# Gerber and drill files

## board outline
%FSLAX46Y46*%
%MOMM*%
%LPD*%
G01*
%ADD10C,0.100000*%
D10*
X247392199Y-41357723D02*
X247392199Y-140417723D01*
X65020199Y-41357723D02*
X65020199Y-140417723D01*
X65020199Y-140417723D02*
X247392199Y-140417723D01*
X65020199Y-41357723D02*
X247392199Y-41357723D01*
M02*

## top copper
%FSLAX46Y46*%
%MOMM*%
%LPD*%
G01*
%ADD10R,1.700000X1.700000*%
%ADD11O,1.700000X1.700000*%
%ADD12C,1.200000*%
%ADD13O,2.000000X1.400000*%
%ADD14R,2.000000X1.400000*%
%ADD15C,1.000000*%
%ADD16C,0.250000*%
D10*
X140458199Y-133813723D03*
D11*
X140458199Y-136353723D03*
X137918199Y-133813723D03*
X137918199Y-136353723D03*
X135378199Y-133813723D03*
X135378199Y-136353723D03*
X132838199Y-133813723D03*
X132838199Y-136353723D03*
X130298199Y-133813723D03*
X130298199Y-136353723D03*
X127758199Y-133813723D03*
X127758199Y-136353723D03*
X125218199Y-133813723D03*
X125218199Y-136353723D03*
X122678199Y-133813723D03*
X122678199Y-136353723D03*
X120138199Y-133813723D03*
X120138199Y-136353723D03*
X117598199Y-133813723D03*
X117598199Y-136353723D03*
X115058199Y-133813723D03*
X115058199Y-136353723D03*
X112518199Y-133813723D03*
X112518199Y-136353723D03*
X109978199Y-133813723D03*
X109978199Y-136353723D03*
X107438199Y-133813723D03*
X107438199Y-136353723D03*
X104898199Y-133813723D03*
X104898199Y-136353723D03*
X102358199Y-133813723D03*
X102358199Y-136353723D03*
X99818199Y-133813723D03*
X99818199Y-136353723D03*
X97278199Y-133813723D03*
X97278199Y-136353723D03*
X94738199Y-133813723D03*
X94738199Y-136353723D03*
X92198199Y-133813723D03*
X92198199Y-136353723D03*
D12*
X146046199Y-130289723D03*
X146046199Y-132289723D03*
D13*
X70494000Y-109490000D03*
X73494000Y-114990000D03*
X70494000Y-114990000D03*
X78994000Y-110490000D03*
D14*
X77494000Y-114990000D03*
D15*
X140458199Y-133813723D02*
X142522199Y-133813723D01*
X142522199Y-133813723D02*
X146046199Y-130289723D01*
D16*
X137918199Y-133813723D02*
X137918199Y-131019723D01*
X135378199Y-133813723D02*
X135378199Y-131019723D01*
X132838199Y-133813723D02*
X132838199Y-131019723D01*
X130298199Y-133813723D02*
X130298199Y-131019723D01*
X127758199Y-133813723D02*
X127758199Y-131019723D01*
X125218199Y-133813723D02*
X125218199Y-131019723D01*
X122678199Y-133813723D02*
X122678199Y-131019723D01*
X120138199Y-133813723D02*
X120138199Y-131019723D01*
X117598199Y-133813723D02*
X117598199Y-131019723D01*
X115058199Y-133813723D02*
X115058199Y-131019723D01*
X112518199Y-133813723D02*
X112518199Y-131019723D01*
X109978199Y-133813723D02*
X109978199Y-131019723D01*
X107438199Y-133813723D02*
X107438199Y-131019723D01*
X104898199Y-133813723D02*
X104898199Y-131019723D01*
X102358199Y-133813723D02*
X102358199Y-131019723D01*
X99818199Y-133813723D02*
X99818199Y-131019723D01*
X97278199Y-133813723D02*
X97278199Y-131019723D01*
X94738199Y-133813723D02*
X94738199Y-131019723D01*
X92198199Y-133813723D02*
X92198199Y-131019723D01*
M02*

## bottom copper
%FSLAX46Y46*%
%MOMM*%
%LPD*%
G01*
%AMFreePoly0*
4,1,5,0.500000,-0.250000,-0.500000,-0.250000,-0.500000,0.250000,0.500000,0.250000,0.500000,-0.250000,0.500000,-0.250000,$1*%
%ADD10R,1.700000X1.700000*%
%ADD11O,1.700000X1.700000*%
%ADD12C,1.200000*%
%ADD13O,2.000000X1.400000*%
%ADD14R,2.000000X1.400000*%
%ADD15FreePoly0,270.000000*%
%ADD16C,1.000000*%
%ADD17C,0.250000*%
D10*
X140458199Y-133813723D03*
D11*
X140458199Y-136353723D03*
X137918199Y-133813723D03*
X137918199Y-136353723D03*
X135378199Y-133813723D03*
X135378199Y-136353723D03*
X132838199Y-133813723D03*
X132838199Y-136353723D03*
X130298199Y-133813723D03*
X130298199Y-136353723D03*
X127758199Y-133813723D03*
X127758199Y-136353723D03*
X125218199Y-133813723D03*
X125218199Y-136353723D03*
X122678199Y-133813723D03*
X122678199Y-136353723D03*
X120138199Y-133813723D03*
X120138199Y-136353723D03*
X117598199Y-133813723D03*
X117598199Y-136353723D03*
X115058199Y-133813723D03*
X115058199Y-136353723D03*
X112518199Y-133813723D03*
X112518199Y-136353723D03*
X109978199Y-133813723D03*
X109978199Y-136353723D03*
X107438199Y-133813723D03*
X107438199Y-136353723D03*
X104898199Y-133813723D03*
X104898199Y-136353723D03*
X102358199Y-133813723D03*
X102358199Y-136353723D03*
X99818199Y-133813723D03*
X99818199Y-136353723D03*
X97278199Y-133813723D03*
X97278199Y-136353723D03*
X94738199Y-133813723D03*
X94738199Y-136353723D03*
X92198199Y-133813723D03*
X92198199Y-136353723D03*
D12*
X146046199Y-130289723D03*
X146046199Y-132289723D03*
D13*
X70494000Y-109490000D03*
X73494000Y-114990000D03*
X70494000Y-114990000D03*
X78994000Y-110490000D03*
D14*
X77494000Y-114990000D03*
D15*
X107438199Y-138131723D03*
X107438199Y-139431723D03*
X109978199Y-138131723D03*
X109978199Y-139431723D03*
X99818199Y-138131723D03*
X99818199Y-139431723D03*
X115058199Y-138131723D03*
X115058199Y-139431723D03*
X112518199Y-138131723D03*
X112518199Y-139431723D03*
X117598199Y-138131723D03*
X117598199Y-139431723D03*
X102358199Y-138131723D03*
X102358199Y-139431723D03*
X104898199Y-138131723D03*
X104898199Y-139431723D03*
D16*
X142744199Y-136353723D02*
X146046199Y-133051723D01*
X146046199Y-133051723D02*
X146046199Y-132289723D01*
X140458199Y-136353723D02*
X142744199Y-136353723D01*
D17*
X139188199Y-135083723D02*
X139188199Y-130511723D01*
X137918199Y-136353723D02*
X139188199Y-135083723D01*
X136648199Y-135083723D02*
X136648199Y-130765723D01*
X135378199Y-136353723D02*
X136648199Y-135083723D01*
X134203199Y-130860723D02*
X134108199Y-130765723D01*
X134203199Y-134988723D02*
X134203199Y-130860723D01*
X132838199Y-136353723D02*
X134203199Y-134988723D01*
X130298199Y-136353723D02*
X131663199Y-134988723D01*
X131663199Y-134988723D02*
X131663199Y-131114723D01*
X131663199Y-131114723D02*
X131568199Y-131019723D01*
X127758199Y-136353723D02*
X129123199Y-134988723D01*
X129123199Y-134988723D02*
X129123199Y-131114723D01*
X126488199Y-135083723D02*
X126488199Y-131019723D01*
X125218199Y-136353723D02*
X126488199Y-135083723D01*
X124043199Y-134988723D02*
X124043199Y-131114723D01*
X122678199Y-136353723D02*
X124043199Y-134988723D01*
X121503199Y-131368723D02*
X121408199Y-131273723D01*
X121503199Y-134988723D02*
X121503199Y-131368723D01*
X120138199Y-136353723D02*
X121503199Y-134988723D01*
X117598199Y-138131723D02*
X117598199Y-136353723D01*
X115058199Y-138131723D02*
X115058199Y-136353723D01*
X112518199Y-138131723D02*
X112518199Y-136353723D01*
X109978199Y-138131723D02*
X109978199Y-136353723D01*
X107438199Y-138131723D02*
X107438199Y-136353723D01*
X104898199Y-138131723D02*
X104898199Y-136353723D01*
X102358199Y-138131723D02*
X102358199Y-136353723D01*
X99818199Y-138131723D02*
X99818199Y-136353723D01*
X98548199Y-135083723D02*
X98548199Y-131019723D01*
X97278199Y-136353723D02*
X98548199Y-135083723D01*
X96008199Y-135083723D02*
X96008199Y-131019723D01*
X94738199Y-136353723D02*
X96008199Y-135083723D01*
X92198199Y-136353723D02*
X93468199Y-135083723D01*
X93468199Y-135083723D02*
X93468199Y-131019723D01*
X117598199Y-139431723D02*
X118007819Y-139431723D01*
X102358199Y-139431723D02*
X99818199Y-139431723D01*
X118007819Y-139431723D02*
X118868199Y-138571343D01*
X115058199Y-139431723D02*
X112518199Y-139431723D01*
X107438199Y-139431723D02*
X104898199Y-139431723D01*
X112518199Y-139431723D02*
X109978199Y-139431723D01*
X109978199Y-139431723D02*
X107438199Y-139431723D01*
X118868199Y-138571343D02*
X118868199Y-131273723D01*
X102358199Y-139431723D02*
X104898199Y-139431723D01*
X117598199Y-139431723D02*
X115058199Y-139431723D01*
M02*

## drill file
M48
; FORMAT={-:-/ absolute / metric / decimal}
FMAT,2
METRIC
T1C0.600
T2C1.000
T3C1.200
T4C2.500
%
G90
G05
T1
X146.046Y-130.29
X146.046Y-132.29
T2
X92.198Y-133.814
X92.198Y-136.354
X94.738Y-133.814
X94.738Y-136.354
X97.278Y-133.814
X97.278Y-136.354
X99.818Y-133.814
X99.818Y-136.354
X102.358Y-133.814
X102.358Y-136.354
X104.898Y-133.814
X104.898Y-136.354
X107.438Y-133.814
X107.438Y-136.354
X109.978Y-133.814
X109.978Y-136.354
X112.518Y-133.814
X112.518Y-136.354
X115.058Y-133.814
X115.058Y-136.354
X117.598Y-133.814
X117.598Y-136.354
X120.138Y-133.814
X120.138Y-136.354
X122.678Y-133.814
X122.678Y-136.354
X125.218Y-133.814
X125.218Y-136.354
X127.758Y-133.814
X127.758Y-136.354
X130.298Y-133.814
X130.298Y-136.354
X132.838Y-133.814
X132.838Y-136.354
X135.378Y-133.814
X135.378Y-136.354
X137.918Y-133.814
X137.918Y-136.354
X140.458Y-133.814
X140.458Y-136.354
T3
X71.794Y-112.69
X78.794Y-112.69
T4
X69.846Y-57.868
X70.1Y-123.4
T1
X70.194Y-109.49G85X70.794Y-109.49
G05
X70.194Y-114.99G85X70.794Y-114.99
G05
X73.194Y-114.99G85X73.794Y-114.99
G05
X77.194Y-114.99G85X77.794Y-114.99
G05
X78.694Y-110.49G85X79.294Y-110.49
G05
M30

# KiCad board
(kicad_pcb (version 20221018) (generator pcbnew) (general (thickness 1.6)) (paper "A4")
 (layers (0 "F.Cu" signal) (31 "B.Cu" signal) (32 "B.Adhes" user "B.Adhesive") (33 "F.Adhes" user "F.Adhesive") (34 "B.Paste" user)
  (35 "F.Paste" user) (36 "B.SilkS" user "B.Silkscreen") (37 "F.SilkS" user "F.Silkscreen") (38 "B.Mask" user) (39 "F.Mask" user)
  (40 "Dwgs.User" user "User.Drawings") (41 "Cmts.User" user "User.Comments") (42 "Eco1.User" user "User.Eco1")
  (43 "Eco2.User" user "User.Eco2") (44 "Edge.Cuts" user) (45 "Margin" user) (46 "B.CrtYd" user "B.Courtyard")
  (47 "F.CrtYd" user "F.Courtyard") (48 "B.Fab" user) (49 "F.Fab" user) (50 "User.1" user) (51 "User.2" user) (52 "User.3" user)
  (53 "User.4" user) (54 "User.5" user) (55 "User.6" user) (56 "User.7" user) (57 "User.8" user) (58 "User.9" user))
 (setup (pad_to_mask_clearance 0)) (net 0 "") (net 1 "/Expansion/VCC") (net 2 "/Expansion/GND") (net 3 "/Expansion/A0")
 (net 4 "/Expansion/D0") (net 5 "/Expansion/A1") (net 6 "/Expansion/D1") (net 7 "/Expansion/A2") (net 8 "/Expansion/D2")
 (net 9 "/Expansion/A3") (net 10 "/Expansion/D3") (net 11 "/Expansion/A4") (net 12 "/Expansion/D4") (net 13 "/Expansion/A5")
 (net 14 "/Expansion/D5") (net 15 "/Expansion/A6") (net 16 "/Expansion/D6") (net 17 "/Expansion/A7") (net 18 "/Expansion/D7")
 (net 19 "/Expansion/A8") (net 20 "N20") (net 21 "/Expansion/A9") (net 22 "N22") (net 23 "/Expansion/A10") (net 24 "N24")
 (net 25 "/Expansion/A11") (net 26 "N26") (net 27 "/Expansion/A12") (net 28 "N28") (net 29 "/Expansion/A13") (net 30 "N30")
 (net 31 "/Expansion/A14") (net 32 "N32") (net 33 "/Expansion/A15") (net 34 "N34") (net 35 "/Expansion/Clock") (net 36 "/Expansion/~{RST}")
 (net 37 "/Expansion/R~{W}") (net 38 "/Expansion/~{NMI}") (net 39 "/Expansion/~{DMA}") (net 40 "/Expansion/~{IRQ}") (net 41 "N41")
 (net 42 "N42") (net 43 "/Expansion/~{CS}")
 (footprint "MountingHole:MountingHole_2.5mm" (layer "F.Cu") (at 70.100199 123.399723)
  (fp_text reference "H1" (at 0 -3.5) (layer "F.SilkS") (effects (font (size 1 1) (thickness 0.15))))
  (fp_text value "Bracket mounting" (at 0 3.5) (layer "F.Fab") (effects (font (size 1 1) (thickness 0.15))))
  (pad "" np_thru_hole circle (at 0 0) (size 2.5 2.5) (drill 2.5) (layers "*.Cu" "*.Mask")))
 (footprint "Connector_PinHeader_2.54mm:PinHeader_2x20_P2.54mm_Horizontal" (layer "F.Cu") (at 140.458199 133.813723 -90)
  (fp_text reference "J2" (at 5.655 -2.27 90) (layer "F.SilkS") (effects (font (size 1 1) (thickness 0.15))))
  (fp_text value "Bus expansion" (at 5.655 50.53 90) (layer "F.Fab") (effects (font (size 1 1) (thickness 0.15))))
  (pad "1" thru_hole rect (at 0 0 270) (size 1.7 1.7) (drill 1) (layers "*.Cu" "*.Mask") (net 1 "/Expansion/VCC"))
  (pad "2" thru_hole oval (at 2.54 0 270) (size 1.7 1.7) (drill 1) (layers "*.Cu" "*.Mask") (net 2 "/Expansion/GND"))
  (pad "3" thru_hole oval (at 0 2.54 270) (size 1.7 1.7) (drill 1) (layers "*.Cu" "*.Mask") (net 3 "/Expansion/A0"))
  (pad "4" thru_hole oval (at 2.54 2.54 270) (size 1.7 1.7) (drill 1) (layers "*.Cu" "*.Mask") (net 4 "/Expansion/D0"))
  (pad "5" thru_hole oval (at 0 5.08 270) (size 1.7 1.7) (drill 1) (layers "*.Cu" "*.Mask") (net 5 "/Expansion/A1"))
  (pad "6" thru_hole oval (at 2.54 5.08 270) (size 1.7 1.7) (drill 1) (layers "*.Cu" "*.Mask") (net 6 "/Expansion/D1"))
  (pad "7" thru_hole oval (at 0 7.62 270) (size 1.7 1.7) (drill 1) (layers "*.Cu" "*.Mask") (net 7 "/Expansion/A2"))
  (pad "8" thru_hole oval (at 2.54 7.62 270) (size 1.7 1.7) (drill 1) (layers "*.Cu" "*.Mask") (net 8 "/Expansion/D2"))
  (pad "9" thru_hole oval (at 0 10.16 270) (size 1.7 1.7) (drill 1) (layers "*.Cu" "*.Mask") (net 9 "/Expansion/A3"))
  (pad "10" thru_hole oval (at 2.54 10.16 270) (size 1.7 1.7) (drill 1) (layers "*.Cu" "*.Mask") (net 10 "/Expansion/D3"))
  (pad "11" thru_hole oval (at 0 12.7 270) (size 1.7 1.7) (drill 1) (layers "*.Cu" "*.Mask") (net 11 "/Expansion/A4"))
  (pad "12" thru_hole oval (at 2.54 12.7 270) (size 1.7 1.7) (drill 1) (layers "*.Cu" "*.Mask") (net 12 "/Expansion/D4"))
  (pad "13" thru_hole oval (at 0 15.24 270) (size 1.7 1.7) (drill 1) (layers "*.Cu" "*.Mask") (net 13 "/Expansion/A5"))
  (pad "14" thru_hole oval (at 2.54 15.24 270) (size 1.7 1.7) (drill 1) (layers "*.Cu" "*.Mask") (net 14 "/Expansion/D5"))
  (pad "15" thru_hole oval (at 0 17.78 270) (size 1.7 1.7) (drill 1) (layers "*.Cu" "*.Mask") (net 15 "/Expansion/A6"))
  (pad "16" thru_hole oval (at 2.54 17.78 270) (size 1.7 1.7) (drill 1) (layers "*.Cu" "*.Mask") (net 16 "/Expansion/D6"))
  (pad "17" thru_hole oval (at 0 20.32 270) (size 1.7 1.7) (drill 1) (layers "*.Cu" "*.Mask") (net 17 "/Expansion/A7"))
  (pad "18" thru_hole oval (at 2.54 20.32 270) (size 1.7 1.7) (drill 1) (layers "*.Cu" "*.Mask") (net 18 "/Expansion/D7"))
  (pad "19" thru_hole oval (at 0 22.86 270) (size 1.7 1.7) (drill 1) (layers "*.Cu" "*.Mask") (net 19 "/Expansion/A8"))
  (pad "20" thru_hole oval (at 2.54 22.86 270) (size 1.7 1.7) (drill 1) (layers "*.Cu" "*.Mask") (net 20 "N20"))
  (pad "21" thru_hole oval (at 0 25.4 270) (size 1.7 1.7) (drill 1) (layers "*.Cu" "*.Mask") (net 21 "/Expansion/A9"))
  (pad "22" thru_hole oval (at 2.54 25.4 270) (size 1.7 1.7) (drill 1) (layers "*.Cu" "*.Mask") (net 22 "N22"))
  (pad "23" thru_hole oval (at 0 27.94 270) (size 1.7 1.7) (drill 1) (layers "*.Cu" "*.Mask") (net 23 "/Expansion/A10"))
  (pad "24" thru_hole oval (at 2.54 27.94 270) (size 1.7 1.7) (drill 1) (layers "*.Cu" "*.Mask") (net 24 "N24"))
  (pad "25" thru_hole oval (at 0 30.48 270) (size 1.7 1.7) (drill 1) (layers "*.Cu" "*.Mask") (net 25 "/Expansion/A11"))
  (pad "26" thru_hole oval (at 2.54 30.48 270) (size 1.7 1.7) (drill 1) (layers "*.Cu" "*.Mask") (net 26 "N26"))
  (pad "27" thru_hole oval (at 0 33.02 270) (size 1.7 1.7) (drill 1) (layers "*.Cu" "*.Mask") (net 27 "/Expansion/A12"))
  (pad "28" thru_hole oval (at 2.54 33.02 270) (size 1.7 1.7) (drill 1) (layers "*.Cu" "*.Mask") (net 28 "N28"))
  (pad "29" thru_hole oval (at 0 35.56 270) (size 1.7 1.7) (drill 1) (layers "*.Cu" "*.Mask") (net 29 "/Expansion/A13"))
  (pad "30" thru_hole oval (at 2.54 35.56 270) (size 1.7 1.7) (drill 1) (layers "*.Cu" "*.Mask") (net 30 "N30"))
  (pad "31" thru_hole oval (at 0 38.1 270) (size 1.7 1.7) (drill 1) (layers "*.Cu" "*.Mask") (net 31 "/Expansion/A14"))
  (pad "32" thru_hole oval (at 2.54 38.1 270) (size 1.7 1.7) (drill 1) (layers "*.Cu" "*.Mask") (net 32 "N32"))
  (pad "33" thru_hole oval (at 0 40.64 270) (size 1.7 1.7) (drill 1) (layers "*.Cu" "*.Mask") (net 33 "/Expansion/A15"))
  (pad "34" thru_hole oval (at 2.54 40.64 270) (size 1.7 1.7) (drill 1) (layers "*.Cu" "*.Mask") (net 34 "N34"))
  (pad "35" thru_hole oval (at 0 43.18 270) (size 1.7 1.7) (drill 1) (layers "*.Cu" "*.Mask") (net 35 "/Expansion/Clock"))
  (pad "36" thru_hole oval (at 2.54 43.18 270) (size 1.7 1.7) (drill 1) (layers "*.Cu" "*.Mask") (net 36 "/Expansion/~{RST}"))
  (pad "37" thru_hole oval (at 0 45.72 270) (size 1.7 1.7) (drill 1) (layers "*.Cu" "*.Mask") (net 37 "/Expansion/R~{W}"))
  (pad "38" thru_hole oval (at 2.54 45.72 270) (size 1.7 1.7) (drill 1) (layers "*.Cu" "*.Mask") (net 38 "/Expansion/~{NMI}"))
  (pad "39" thru_hole oval (at 0 48.26 270) (size 1.7 1.7) (drill 1) (layers "*.Cu" "*.Mask") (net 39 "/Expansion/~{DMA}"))
  (pad "40" thru_hole oval (at 2.54 48.26 270) (size 1.7 1.7) (drill 1) (layers "*.Cu" "*.Mask") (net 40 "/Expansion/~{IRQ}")))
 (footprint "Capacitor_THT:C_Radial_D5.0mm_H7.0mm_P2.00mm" (layer "F.Cu") (at 146.046199 130.289723 -90)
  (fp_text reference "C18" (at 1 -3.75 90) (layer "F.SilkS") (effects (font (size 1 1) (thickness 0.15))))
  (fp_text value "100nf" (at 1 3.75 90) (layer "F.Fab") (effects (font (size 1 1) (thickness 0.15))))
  (pad "1" thru_hole circle (at 0 0 270) (size 1.2 1.2) (drill 0.6) (layers "*.Cu" "*.Mask") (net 1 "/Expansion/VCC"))
  (pad "2" thru_hole circle (at 2 0 270) (size 1.2 1.2) (drill 0.6) (layers "*.Cu" "*.Mask") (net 2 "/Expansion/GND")))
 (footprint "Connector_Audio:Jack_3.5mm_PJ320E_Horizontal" (layer "F.Cu") (at 77.494 114.99 90)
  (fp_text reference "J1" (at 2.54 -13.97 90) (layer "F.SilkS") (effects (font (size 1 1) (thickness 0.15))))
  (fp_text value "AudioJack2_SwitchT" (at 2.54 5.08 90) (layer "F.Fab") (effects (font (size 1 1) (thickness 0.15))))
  (pad "" np_thru_hole circle (at 2.3 -5.7) (size 1.2 1.2) (drill 1.2) (layers "*.Cu" "*.Mask"))
  (pad "" np_thru_hole circle (at 2.3 1.3) (size 1.2 1.2) (drill 1.2) (layers "*.Cu" "*.Mask"))
  (pad "" thru_hole oval (at 5.5 -7) (size 2 1.4) (drill oval 1.2 0.6) (layers "*.Cu" "*.Mask"))
  (pad "R1" thru_hole oval (at 0 -4) (size 2 1.4) (drill oval 1.2 0.6) (layers "*.Cu" "*.Mask"))
  (pad "R2" thru_hole oval (at 0 -7) (size 2 1.4) (drill oval 1.2 0.6) (layers "*.Cu" "*.Mask"))
  (pad "S" thru_hole oval (at 4.5 1.5) (size 2 1.4) (drill oval 1.2 0.6) (layers "*.Cu" "*.Mask") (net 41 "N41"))
  (pad "T" thru_hole rect (at 0 0) (size 2 1.4) (drill oval 1.2 0.6) (layers "*.Cu" "*.Mask") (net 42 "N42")))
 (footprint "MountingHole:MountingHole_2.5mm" (layer "F.Cu") (at 69.846199 57.867723)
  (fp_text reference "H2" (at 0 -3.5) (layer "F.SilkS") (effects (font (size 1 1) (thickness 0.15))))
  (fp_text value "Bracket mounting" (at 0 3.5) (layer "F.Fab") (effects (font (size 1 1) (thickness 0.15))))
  (pad "" np_thru_hole circle (at 0 0) (size 2.5 2.5) (drill 2.5) (layers "*.Cu" "*.Mask")))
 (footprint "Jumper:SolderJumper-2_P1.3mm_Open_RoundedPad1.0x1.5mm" (layer "B.Cu") (at 107.438199 138.781723 -90)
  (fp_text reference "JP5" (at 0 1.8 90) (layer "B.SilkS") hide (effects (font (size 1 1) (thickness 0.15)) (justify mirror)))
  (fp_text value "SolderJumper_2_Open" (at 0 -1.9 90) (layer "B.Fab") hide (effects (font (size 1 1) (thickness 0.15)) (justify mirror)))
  (pad "1" smd custom (at -0.65 0 270) (size 1 0.5) (layers "B.Cu" "B.Mask") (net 28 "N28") (zone_connect 2) (thermal_bridge_angle 45)
   (options (clearance outline) (anchor rect)) (primitives))
  (pad "2" smd custom (at 0.65 0 270) (size 1 0.5) (layers "B.Cu" "B.Mask") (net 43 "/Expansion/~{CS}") (zone_connect 2)
   (thermal_bridge_angle 45) (options (clearance outline) (anchor rect)) (primitives)))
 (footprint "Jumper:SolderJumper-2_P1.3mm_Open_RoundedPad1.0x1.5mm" (layer "B.Cu") (at 109.978199 138.781723 -90)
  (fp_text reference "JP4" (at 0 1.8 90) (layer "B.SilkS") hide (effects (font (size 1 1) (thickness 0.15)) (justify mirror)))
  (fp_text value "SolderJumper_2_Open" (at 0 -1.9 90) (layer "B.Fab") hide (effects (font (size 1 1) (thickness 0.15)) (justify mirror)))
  (pad "1" smd custom (at -0.65 0 270) (size 1 0.5) (layers "B.Cu" "B.Mask") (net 26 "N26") (zone_connect 2) (thermal_bridge_angle 45)
   (options (clearance outline) (anchor rect)) (primitives))
  (pad "2" smd custom (at 0.65 0 270) (size 1 0.5) (layers "B.Cu" "B.Mask") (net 43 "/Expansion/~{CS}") (zone_connect 2)
   (thermal_bridge_angle 45) (options (clearance outline) (anchor rect)) (primitives)))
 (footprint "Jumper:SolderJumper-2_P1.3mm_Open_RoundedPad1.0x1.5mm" (layer "B.Cu") (at 99.818199 138.781723 -90)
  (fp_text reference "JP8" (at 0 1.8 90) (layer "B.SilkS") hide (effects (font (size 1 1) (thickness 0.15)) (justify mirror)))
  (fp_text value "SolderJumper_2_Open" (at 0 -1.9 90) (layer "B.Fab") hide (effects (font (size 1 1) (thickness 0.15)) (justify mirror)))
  (pad "1" smd custom (at -0.65 0 270) (size 1 0.5) (layers "B.Cu" "B.Mask") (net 34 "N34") (zone_connect 2) (thermal_bridge_angle 45)
   (options (clearance outline) (anchor rect)) (primitives))
  (pad "2" smd custom (at 0.65 0 270) (size 1 0.5) (layers "B.Cu" "B.Mask") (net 43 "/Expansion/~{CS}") (zone_connect 2)
   (thermal_bridge_angle 45) (options (clearance outline) (anchor rect)) (primitives)))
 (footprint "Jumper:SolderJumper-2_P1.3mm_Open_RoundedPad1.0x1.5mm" (layer "B.Cu") (at 115.058199 138.781723 -90)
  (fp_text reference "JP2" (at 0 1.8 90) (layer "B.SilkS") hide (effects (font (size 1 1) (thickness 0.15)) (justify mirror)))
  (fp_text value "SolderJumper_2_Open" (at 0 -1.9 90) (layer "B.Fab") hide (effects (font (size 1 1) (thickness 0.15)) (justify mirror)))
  (pad "1" smd custom (at -0.65 0 270) (size 1 0.5) (layers "B.Cu" "B.Mask") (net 22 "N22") (zone_connect 2) (thermal_bridge_angle 45)
   (options (clearance outline) (anchor rect)) (primitives))
  (pad "2" smd custom (at 0.65 0 270) (size 1 0.5) (layers "B.Cu" "B.Mask") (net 43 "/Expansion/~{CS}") (zone_connect 2)
   (thermal_bridge_angle 45) (options (clearance outline) (anchor rect)) (primitives)))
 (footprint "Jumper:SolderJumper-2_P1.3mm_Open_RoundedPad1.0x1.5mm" (layer "B.Cu") (at 112.518199 138.781723 -90)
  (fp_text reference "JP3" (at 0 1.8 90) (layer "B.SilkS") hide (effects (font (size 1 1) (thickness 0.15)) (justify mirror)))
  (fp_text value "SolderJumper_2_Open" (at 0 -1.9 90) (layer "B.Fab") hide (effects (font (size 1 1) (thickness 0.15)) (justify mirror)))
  (pad "1" smd custom (at -0.65 0 270) (size 1 0.5) (layers "B.Cu" "B.Mask") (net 24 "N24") (zone_connect 2) (thermal_bridge_angle 45)
   (options (clearance outline) (anchor rect)) (primitives))
  (pad "2" smd custom (at 0.65 0 270) (size 1 0.5) (layers "B.Cu" "B.Mask") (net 43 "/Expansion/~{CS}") (zone_connect 2)
   (thermal_bridge_angle 45) (options (clearance outline) (anchor rect)) (primitives)))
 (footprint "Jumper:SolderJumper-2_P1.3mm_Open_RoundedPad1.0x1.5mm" (layer "B.Cu") (at 117.598199 138.781723 -90)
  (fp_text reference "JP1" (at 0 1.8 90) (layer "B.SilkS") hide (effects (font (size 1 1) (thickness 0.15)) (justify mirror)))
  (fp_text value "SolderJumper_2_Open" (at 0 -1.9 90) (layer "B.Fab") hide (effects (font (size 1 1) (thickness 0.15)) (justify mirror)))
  (pad "1" smd custom (at -0.65 0 270) (size 1 0.5) (layers "B.Cu" "B.Mask") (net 20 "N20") (zone_connect 2) (thermal_bridge_angle 45)
   (options (clearance outline) (anchor rect)) (primitives))
  (pad "2" smd custom (at 0.65 0 270) (size 1 0.5) (layers "B.Cu" "B.Mask") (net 43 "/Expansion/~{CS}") (zone_connect 2)
   (thermal_bridge_angle 45) (options (clearance outline) (anchor rect)) (primitives)))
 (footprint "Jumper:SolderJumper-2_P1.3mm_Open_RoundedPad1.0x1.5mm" (layer "B.Cu") (at 102.358199 138.781723 -90)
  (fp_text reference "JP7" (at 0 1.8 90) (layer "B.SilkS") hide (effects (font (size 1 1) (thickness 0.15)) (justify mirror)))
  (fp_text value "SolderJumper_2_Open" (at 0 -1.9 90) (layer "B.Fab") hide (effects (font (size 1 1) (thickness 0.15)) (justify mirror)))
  (pad "1" smd custom (at -0.65 0 270) (size 1 0.5) (layers "B.Cu" "B.Mask") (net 32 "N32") (zone_connect 2) (thermal_bridge_angle 45)
   (options (clearance outline) (anchor rect)) (primitives))
  (pad "2" smd custom (at 0.65 0 270) (size 1 0.5) (layers "B.Cu" "B.Mask") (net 43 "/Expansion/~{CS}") (zone_connect 2)
   (thermal_bridge_angle 45) (options (clearance outline) (anchor rect)) (primitives)))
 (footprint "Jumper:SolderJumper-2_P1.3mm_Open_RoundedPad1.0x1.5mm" (layer "B.Cu") (at 104.898199 138.781723 -90)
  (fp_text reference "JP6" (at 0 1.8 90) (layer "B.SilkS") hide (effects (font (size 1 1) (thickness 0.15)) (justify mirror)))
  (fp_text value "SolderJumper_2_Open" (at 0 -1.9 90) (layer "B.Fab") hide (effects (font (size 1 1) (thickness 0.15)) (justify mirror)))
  (pad "1" smd custom (at -0.65 0 270) (size 1 0.5) (layers "B.Cu" "B.Mask") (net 30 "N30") (zone_connect 2) (thermal_bridge_angle 45)
   (options (clearance outline) (anchor rect)) (primitives))
  (pad "2" smd custom (at 0.65 0 270) (size 1 0.5) (layers "B.Cu" "B.Mask") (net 43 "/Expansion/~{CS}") (zone_connect 2)
   (thermal_bridge_angle 45) (options (clearance outline) (anchor rect)) (primitives)))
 (gr_line (start 247.392199 41.357723) (end 247.392199 140.417723) (stroke (width 0.1) (type default)) (layer "Edge.Cuts"))
 (gr_line (start 65.020199 41.357723) (end 65.020199 140.417723) (stroke (width 0.1) (type default)) (layer "Edge.Cuts"))
 (gr_line (start 65.020199 140.417723) (end 247.392199 140.417723) (stroke (width 0.1) (type default)) (layer "Edge.Cuts"))
 (gr_line (start 65.020199 41.357723) (end 247.392199 41.357723) (stroke (width 0.1) (type default)) (layer "Edge.Cuts"))
 (segment (start 140.458199 133.813723) (end 142.522199 133.813723) (width 1) (layer "F.Cu") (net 1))
 (segment (start 142.522199 133.813723) (end 146.046199 130.289723) (width 1) (layer "F.Cu") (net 1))
 (segment (start 142.744199 136.353723) (end 146.046199 133.051723) (width 1) (layer "B.Cu") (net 2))
 (segment (start 146.046199 133.051723) (end 146.046199 132.289723) (width 1) (layer "B.Cu") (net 2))
 (segment (start 140.458199 136.353723) (end 142.744199 136.353723) (width 1) (layer "B.Cu") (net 2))
 (segment (start 137.918199 133.813723) (end 137.918199 131.019723) (width 0.25) (layer "F.Cu") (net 3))
 (segment (start 139.188199 135.083723) (end 139.188199 130.511723) (width 0.25) (layer "B.Cu") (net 4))
 (segment (start 137.918199 136.353723) (end 139.188199 135.083723) (width 0.25) (layer "B.Cu") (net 4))
 (segment (start 135.378199 133.813723) (end 135.378199 131.019723) (width 0.25) (layer "F.Cu") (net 5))
 (segment (start 136.648199 135.083723) (end 136.648199 130.765723) (width 0.25) (layer "B.Cu") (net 6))
 (segment (start 135.378199 136.353723) (end 136.648199 135.083723) (width 0.25) (layer "B.Cu") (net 6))
 (segment (start 132.838199 133.813723) (end 132.838199 131.019723) (width 0.25) (layer "F.Cu") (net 7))
 (segment (start 134.203199 130.860723) (end 134.108199 130.765723) (width 0.25) (layer "B.Cu") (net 8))
 (segment (start 134.203199 134.988723) (end 134.203199 130.860723) (width 0.25) (layer "B.Cu") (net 8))
 (segment (start 132.838199 136.353723) (end 134.203199 134.988723) (width 0.25) (layer "B.Cu") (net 8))
 (segment (start 130.298199 133.813723) (end 130.298199 131.019723) (width 0.25) (layer "F.Cu") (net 9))
 (segment (start 130.298199 136.353723) (end 131.663199 134.988723) (width 0.25) (layer "B.Cu") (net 10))
 (segment (start 131.663199 134.988723) (end 131.663199 131.114723) (width 0.25) (layer "B.Cu") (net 10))
 (segment (start 131.663199 131.114723) (end 131.568199 131.019723) (width 0.25) (layer "B.Cu") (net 10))
 (segment (start 127.758199 133.813723) (end 127.758199 131.019723) (width 0.25) (layer "F.Cu") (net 11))
 (segment (start 127.758199 136.353723) (end 129.123199 134.988723) (width 0.25) (layer "B.Cu") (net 12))
 (segment (start 129.123199 134.988723) (end 129.123199 131.114723) (width 0.25) (layer "B.Cu") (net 12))
 (segment (start 125.218199 133.813723) (end 125.218199 131.019723) (width 0.25) (layer "F.Cu") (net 13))
 (segment (start 126.488199 135.083723) (end 126.488199 131.019723) (width 0.25) (layer "B.Cu") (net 14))
 (segment (start 125.218199 136.353723) (end 126.488199 135.083723) (width 0.25) (layer "B.Cu") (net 14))
 (segment (start 122.678199 133.813723) (end 122.678199 131.019723) (width 0.25) (layer "F.Cu") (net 15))
 (segment (start 124.043199 134.988723) (end 124.043199 131.114723) (width 0.25) (layer "B.Cu") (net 16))
 (segment (start 122.678199 136.353723) (end 124.043199 134.988723) (width 0.25) (layer "B.Cu") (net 16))
 (segment (start 120.138199 133.813723) (end 120.138199 131.019723) (width 0.25) (layer "F.Cu") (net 17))
 (segment (start 121.503199 131.368723) (end 121.408199 131.273723) (width 0.25) (layer "B.Cu") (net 18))
 (segment (start 121.503199 134.988723) (end 121.503199 131.368723) (width 0.25) (layer "B.Cu") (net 18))
 (segment (start 120.138199 136.353723) (end 121.503199 134.988723) (width 0.25) (layer "B.Cu") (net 18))
 (segment (start 117.598199 133.813723) (end 117.598199 131.019723) (width 0.25) (layer "F.Cu") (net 19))
 (segment (start 117.598199 138.131723) (end 117.598199 136.353723) (width 0.25) (layer "B.Cu") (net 20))
 (segment (start 115.058199 133.813723) (end 115.058199 131.019723) (width 0.25) (layer "F.Cu") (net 21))
 (segment (start 115.058199 138.131723) (end 115.058199 136.353723) (width 0.25) (layer "B.Cu") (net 22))
 (segment (start 112.518199 133.813723) (end 112.518199 131.019723) (width 0.25) (layer "F.Cu") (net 23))
 (segment (start 112.518199 138.131723) (end 112.518199 136.353723) (width 0.25) (layer "B.Cu") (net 24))
 (segment (start 109.978199 133.813723) (end 109.978199 131.019723) (width 0.25) (layer "F.Cu") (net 25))
 (segment (start 109.978199 138.131723) (end 109.978199 136.353723) (width 0.25) (layer "B.Cu") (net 26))
 (segment (start 107.438199 133.813723) (end 107.438199 131.019723) (width 0.25) (layer "F.Cu") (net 27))
 (segment (start 107.438199 138.131723) (end 107.438199 136.353723) (width 0.25) (layer "B.Cu") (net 28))
 (segment (start 104.898199 133.813723) (end 104.898199 131.019723) (width 0.25) (layer "F.Cu") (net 29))
 (segment (start 104.898199 138.131723) (end 104.898199 136.353723) (width 0.25) (layer "B.Cu") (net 30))
 (segment (start 102.358199 133.813723) (end 102.358199 131.019723) (width 0.25) (layer "F.Cu") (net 31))
 (segment (start 102.358199 138.131723) (end 102.358199 136.353723) (width 0.25) (layer "B.Cu") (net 32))
 (segment (start 99.818199 133.813723) (end 99.818199 131.019723) (width 0.25) (layer "F.Cu") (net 33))
 (segment (start 99.818199 138.131723) (end 99.818199 136.353723) (width 0.25) (layer "B.Cu") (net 34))
 (segment (start 97.278199 133.813723) (end 97.278199 131.019723) (width 0.25) (layer "F.Cu") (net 35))
 (segment (start 98.548199 135.083723) (end 98.548199 131.019723) (width 0.25) (layer "B.Cu") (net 36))
 (segment (start 97.278199 136.353723) (end 98.548199 135.083723) (width 0.25) (layer "B.Cu") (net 36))
 (segment (start 94.738199 133.813723) (end 94.738199 131.019723) (width 0.25) (layer "F.Cu") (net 37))
 (segment (start 96.008199 135.083723) (end 96.008199 131.019723) (width 0.25) (layer "B.Cu") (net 38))
 (segment (start 94.738199 136.353723) (end 96.008199 135.083723) (width 0.25) (layer "B.Cu") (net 38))
 (segment (start 92.198199 133.813723) (end 92.198199 131.019723) (width 0.25) (layer "F.Cu") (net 39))
 (segment (start 92.198199 136.353723) (end 93.468199 135.083723) (width 0.25) (layer "B.Cu") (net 40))
 (segment (start 93.468199 135.083723) (end 93.468199 131.019723) (width 0.25) (layer "B.Cu") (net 40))
 (segment (start 117.598199 139.431723) (end 118.007819 139.431723) (width 0.25) (layer "B.Cu") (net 43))
 (segment (start 102.358199 139.431723) (end 99.818199 139.431723) (width 0.25) (layer "B.Cu") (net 43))
 (segment (start 118.007819 139.431723) (end 118.868199 138.571343) (width 0.25) (layer "B.Cu") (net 43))
 (segment (start 115.058199 139.431723) (end 112.518199 139.431723) (width 0.25) (layer "B.Cu") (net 43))
 (segment (start 107.438199 139.431723) (end 104.898199 139.431723) (width 0.25) (layer "B.Cu") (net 43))
 (segment (start 112.518199 139.431723) (end 109.978199 139.431723) (width 0.25) (layer "B.Cu") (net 43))
 (segment (start 109.978199 139.431723) (end 107.438199 139.431723) (width 0.25) (layer "B.Cu") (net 43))
 (segment (start 118.868199 138.571343) (end 118.868199 131.273723) (width 0.25) (layer "B.Cu") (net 43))
 (segment (start 102.358199 139.431723) (end 104.898199 139.431723) (width 0.25) (layer "B.Cu") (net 43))
 (segment (start 117.598199 139.431723) (end 115.058199 139.431723) (width 0.25) (layer "B.Cu") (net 43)))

